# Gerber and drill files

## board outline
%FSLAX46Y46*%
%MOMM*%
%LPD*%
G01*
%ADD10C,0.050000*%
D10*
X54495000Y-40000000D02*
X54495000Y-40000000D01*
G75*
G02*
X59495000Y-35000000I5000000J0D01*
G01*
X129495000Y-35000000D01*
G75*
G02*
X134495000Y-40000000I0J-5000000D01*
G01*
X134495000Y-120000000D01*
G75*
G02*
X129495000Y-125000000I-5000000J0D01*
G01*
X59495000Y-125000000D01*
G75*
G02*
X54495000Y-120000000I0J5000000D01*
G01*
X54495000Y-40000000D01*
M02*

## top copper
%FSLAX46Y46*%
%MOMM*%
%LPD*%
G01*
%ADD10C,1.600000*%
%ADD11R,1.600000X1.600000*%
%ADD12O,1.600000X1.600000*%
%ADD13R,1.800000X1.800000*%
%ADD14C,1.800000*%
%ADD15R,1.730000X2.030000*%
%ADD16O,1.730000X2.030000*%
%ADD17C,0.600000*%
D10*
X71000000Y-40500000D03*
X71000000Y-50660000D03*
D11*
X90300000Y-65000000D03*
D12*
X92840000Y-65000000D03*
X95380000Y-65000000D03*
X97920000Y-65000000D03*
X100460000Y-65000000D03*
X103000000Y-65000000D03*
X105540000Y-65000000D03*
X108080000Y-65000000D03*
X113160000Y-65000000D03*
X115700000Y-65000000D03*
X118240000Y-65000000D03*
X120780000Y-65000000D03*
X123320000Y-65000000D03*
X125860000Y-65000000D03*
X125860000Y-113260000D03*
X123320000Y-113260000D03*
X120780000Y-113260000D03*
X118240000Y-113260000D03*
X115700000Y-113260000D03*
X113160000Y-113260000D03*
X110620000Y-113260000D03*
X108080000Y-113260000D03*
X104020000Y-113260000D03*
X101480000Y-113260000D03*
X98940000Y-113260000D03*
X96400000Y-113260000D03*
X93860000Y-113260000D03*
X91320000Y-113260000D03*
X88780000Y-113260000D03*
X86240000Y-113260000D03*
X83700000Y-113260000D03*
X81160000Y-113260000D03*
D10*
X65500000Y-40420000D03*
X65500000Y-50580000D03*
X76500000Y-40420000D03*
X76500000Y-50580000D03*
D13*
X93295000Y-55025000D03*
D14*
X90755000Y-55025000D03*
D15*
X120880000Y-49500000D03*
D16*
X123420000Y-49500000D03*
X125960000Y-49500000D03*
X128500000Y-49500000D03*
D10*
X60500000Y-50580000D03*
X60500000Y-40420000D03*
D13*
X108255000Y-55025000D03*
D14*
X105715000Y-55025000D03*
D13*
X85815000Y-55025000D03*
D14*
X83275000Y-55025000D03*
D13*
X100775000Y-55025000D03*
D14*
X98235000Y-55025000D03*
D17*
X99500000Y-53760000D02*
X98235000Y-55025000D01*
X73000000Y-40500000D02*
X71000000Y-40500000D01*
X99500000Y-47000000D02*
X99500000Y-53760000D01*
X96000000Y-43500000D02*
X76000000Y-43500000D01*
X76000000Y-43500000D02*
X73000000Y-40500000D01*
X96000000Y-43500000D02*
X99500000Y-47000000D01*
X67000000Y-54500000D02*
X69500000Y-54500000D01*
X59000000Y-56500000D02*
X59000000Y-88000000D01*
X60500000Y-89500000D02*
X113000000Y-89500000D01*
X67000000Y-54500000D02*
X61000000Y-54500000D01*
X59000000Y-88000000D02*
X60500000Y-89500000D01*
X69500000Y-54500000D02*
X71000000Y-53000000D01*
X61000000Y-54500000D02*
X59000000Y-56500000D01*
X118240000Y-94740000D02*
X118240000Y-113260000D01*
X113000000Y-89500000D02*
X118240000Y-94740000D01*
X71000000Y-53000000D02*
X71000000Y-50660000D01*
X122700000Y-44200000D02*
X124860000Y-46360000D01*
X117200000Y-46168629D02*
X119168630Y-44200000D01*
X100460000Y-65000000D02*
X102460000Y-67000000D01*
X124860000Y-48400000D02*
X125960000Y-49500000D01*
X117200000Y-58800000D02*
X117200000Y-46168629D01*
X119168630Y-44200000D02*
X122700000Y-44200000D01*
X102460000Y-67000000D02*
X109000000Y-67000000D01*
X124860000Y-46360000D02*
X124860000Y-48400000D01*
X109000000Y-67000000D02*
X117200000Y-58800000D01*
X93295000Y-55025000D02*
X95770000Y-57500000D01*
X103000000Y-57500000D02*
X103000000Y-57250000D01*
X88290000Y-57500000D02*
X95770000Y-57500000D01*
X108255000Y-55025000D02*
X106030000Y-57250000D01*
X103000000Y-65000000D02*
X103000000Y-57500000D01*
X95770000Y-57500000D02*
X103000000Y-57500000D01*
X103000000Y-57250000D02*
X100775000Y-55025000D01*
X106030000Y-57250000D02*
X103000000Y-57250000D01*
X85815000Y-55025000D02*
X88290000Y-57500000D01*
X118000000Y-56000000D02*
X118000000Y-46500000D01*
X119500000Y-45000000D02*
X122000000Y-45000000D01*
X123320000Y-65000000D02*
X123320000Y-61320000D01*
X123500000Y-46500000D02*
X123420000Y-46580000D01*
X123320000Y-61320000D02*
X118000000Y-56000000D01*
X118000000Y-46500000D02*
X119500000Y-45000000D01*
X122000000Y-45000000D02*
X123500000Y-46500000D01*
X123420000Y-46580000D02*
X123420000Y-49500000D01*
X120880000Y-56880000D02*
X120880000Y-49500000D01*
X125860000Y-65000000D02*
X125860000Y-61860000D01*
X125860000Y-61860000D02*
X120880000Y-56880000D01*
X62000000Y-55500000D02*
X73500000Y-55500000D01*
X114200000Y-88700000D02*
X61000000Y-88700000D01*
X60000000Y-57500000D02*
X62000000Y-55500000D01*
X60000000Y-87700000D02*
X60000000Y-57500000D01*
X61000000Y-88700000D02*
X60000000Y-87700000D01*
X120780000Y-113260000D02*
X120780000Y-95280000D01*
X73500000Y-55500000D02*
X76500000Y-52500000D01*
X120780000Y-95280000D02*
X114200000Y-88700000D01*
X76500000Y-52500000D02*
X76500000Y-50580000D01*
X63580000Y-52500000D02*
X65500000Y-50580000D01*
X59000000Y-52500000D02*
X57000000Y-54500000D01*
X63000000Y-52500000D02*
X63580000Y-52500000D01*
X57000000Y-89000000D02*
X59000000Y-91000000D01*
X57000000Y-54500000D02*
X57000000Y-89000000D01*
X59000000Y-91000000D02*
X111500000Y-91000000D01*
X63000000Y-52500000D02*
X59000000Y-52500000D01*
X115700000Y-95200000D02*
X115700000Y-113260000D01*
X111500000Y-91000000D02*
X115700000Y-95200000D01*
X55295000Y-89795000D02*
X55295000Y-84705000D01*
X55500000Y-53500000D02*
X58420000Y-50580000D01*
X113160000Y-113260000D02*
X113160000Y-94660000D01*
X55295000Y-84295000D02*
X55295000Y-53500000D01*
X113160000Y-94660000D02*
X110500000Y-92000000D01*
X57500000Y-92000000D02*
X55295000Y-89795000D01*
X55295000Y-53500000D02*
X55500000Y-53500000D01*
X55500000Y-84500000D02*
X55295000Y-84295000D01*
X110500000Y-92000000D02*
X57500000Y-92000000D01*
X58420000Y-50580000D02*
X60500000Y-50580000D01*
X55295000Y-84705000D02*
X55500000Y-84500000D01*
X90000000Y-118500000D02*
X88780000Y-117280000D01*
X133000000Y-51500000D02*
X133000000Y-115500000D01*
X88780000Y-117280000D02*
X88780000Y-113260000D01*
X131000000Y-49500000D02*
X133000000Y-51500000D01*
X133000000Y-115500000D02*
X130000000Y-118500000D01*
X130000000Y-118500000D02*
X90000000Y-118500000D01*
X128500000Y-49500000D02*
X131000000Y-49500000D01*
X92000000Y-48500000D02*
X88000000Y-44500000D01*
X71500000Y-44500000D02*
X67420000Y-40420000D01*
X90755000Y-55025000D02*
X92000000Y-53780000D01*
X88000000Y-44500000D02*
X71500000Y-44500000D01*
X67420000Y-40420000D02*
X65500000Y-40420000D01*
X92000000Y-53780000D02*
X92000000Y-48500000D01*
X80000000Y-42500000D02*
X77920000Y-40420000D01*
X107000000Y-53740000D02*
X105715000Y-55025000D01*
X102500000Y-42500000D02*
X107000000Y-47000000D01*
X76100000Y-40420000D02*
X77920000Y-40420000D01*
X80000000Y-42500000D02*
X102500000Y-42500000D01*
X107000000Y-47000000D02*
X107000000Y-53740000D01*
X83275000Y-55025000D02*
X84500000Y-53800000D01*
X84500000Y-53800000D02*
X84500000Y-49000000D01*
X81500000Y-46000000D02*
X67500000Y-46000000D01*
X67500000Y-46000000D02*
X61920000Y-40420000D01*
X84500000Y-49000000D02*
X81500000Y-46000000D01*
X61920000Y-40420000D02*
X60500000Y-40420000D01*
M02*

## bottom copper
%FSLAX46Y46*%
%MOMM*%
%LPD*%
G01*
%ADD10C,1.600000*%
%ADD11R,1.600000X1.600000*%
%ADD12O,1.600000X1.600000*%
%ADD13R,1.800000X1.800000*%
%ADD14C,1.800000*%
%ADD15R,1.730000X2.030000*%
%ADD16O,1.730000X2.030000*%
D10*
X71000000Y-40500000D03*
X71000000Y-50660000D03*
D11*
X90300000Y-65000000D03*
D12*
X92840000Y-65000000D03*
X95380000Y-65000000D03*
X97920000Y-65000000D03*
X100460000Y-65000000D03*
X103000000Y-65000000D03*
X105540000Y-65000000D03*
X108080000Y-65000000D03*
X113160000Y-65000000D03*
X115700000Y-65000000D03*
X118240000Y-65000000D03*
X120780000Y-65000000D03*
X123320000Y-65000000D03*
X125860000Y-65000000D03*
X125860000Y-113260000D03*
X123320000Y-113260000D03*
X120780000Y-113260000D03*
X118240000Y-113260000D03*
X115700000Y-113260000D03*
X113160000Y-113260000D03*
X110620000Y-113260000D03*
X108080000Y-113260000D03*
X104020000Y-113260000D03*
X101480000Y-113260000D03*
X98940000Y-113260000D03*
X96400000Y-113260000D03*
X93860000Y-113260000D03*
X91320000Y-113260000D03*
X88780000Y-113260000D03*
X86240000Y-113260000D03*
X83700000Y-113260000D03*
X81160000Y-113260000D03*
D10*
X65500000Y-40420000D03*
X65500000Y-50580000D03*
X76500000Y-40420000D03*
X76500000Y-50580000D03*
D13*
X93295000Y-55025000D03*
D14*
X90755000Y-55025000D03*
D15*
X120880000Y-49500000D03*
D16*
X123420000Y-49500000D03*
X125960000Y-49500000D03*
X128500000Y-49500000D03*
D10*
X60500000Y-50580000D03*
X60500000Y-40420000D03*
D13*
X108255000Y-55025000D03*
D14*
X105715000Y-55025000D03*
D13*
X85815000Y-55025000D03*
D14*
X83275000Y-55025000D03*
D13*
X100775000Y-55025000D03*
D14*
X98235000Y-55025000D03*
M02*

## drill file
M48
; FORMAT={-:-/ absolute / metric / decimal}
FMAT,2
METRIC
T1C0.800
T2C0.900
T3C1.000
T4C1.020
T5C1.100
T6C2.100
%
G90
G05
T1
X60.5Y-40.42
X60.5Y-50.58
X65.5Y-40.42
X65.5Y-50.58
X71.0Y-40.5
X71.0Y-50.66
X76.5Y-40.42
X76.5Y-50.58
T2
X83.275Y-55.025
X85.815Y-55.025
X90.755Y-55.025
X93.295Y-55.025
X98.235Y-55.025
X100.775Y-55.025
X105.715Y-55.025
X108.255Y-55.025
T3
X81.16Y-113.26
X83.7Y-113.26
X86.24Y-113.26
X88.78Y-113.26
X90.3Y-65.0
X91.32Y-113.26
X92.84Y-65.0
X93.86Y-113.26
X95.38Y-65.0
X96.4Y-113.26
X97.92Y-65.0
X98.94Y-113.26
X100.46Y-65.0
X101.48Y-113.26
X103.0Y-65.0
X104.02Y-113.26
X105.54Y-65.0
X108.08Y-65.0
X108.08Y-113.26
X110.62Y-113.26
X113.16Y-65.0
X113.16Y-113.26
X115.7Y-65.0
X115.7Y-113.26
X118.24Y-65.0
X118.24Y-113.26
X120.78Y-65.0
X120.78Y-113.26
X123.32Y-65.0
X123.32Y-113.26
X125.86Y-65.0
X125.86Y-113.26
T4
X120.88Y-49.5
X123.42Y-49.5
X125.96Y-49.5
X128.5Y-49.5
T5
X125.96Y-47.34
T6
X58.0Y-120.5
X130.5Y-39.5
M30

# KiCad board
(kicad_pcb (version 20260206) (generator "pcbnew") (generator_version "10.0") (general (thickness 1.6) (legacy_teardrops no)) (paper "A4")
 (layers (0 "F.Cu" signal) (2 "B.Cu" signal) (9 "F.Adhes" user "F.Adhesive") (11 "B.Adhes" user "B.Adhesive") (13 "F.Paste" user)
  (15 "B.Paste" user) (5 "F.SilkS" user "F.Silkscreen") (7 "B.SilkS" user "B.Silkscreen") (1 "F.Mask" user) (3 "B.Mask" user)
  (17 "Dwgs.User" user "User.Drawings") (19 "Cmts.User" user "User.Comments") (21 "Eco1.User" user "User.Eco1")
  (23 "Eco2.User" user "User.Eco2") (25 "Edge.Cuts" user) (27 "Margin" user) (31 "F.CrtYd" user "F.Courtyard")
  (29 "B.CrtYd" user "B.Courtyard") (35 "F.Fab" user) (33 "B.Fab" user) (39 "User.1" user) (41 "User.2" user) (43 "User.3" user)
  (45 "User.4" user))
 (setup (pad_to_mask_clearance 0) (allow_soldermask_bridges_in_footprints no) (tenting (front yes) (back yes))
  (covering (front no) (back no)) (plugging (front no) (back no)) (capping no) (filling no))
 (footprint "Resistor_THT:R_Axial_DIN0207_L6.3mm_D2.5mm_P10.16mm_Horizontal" (layer "F.Cu") (at 71 40.5 -90)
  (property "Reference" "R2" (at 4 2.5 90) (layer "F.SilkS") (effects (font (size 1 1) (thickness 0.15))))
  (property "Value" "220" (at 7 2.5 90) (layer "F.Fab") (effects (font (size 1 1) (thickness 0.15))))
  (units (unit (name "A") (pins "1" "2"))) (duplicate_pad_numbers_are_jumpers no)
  (pad "1" thru_hole circle (at 0 0 270) (size 1.6 1.6) (drill 0.8) (layers "*.Cu" "*.Mask") (remove_unused_layers no) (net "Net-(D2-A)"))
  (pad "2" thru_hole circle (at 10.16 0 270) (size 1.6 1.6) (drill 0.8) (layers "*.Cu" "*.Mask") (remove_unused_layers no)
   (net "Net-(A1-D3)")))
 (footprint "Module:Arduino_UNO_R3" (layer "F.Cu") (at 90.3 65)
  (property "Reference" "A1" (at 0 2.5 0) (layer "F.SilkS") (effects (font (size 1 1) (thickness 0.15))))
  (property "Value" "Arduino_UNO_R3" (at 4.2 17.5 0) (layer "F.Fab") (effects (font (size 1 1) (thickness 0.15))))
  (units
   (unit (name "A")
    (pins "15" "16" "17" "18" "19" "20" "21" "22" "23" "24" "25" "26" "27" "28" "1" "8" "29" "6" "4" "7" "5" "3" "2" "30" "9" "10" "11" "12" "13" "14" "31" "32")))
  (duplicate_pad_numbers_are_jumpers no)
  (pad "1" thru_hole rect (at 0 0 90) (size 1.6 1.6) (drill 1) (layers "*.Cu" "*.Mask") (remove_unused_layers no)
   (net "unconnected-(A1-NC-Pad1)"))
  (pad "2" thru_hole oval (at 2.54 0 90) (size 1.6 1.6) (drill 1) (layers "*.Cu" "*.Mask") (remove_unused_layers no)
   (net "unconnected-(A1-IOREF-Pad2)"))
  (pad "3" thru_hole oval (at 5.08 0 90) (size 1.6 1.6) (drill 1) (layers "*.Cu" "*.Mask") (remove_unused_layers no)
   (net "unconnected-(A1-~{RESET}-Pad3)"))
  (pad "4" thru_hole oval (at 7.62 0 90) (size 1.6 1.6) (drill 1) (layers "*.Cu" "*.Mask") (remove_unused_layers no)
   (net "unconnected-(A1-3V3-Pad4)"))
  (pad "5" thru_hole oval (at 10.16 0 90) (size 1.6 1.6) (drill 1) (layers "*.Cu" "*.Mask") (remove_unused_layers no) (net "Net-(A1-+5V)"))
  (pad "6" thru_hole oval (at 12.7 0 90) (size 1.6 1.6) (drill 1) (layers "*.Cu" "*.Mask") (remove_unused_layers no) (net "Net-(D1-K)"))
  (pad "7" thru_hole oval (at 15.24 0 90) (size 1.6 1.6) (drill 1) (layers "*.Cu" "*.Mask") (remove_unused_layers no)
   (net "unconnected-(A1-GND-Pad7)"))
  (pad "8" thru_hole oval (at 17.78 0 90) (size 1.6 1.6) (drill 1) (layers "*.Cu" "*.Mask") (remove_unused_layers no)
   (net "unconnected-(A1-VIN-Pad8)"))
  (pad "9" thru_hole oval (at 22.86 0 90) (size 1.6 1.6) (drill 1) (layers "*.Cu" "*.Mask") (remove_unused_layers no)
   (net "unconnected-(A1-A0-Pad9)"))
  (pad "10" thru_hole oval (at 25.4 0 90) (size 1.6 1.6) (drill 1) (layers "*.Cu" "*.Mask") (remove_unused_layers no)
   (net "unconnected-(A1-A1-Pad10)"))
  (pad "11" thru_hole oval (at 27.94 0 90) (size 1.6 1.6) (drill 1) (layers "*.Cu" "*.Mask") (remove_unused_layers no)
   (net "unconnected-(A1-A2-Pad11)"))
  (pad "12" thru_hole oval (at 30.48 0 90) (size 1.6 1.6) (drill 1) (layers "*.Cu" "*.Mask") (remove_unused_layers no)
   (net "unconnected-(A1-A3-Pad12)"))
  (pad "13" thru_hole oval (at 33.02 0 90) (size 1.6 1.6) (drill 1) (layers "*.Cu" "*.Mask") (remove_unused_layers no)
   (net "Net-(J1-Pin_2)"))
  (pad "14" thru_hole oval (at 35.56 0 90) (size 1.6 1.6) (drill 1) (layers "*.Cu" "*.Mask") (remove_unused_layers no)
   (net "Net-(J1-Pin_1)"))
  (pad "15" thru_hole oval (at 35.56 48.26 90) (size 1.6 1.6) (drill 1) (layers "*.Cu" "*.Mask") (remove_unused_layers no)
   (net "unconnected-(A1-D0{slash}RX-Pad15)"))
  (pad "16" thru_hole oval (at 33.02 48.26 90) (size 1.6 1.6) (drill 1) (layers "*.Cu" "*.Mask") (remove_unused_layers no)
   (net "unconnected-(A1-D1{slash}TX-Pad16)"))
  (pad "17" thru_hole oval (at 30.48 48.26 90) (size 1.6 1.6) (drill 1) (layers "*.Cu" "*.Mask") (remove_unused_layers no)
   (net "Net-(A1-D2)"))
  (pad "18" thru_hole oval (at 27.94 48.26 90) (size 1.6 1.6) (drill 1) (layers "*.Cu" "*.Mask") (remove_unused_layers no)
   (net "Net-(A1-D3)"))
  (pad "19" thru_hole oval (at 25.4 48.26 90) (size 1.6 1.6) (drill 1) (layers "*.Cu" "*.Mask") (remove_unused_layers no)
   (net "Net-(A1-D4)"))
  (pad "20" thru_hole oval (at 22.86 48.26 90) (size 1.6 1.6) (drill 1) (layers "*.Cu" "*.Mask") (remove_unused_layers no)
   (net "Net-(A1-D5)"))
  (pad "21" thru_hole oval (at 20.32 48.26 90) (size 1.6 1.6) (drill 1) (layers "*.Cu" "*.Mask") (remove_unused_layers no)
   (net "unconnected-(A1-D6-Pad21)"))
  (pad "22" thru_hole oval (at 17.78 48.26 90) (size 1.6 1.6) (drill 1) (layers "*.Cu" "*.Mask") (remove_unused_layers no)
   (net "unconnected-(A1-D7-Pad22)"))
  (pad "23" thru_hole oval (at 13.72 48.26 90) (size 1.6 1.6) (drill 1) (layers "*.Cu" "*.Mask") (remove_unused_layers no)
   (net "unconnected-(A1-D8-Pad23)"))
  (pad "24" thru_hole oval (at 11.18 48.26 90) (size 1.6 1.6) (drill 1) (layers "*.Cu" "*.Mask") (remove_unused_layers no)
   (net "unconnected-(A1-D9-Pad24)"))
  (pad "25" thru_hole oval (at 8.64 48.26 90) (size 1.6 1.6) (drill 1) (layers "*.Cu" "*.Mask") (remove_unused_layers no)
   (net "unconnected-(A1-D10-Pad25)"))
  (pad "26" thru_hole oval (at 6.1 48.26 90) (size 1.6 1.6) (drill 1) (layers "*.Cu" "*.Mask") (remove_unused_layers no)
   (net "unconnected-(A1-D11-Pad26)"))
  (pad "27" thru_hole oval (at 3.56 48.26 90) (size 1.6 1.6) (drill 1) (layers "*.Cu" "*.Mask") (remove_unused_layers no)
   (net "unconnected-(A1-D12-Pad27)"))
  (pad "28" thru_hole oval (at 1.02 48.26 90) (size 1.6 1.6) (drill 1) (layers "*.Cu" "*.Mask") (remove_unused_layers no)
   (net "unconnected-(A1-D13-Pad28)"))
  (pad "29" thru_hole oval (at -1.52 48.26 90) (size 1.6 1.6) (drill 1) (layers "*.Cu" "*.Mask") (remove_unused_layers no)
   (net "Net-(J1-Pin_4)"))
  (pad "30" thru_hole oval (at -4.06 48.26 90) (size 1.6 1.6) (drill 1) (layers "*.Cu" "*.Mask") (remove_unused_layers no)
   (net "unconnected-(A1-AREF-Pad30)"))
  (pad "31" thru_hole oval (at -6.6 48.26 90) (size 1.6 1.6) (drill 1) (layers "*.Cu" "*.Mask") (remove_unused_layers no)
   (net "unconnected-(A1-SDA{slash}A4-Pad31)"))
  (pad "32" thru_hole oval (at -9.14 48.26 90) (size 1.6 1.6) (drill 1) (layers "*.Cu" "*.Mask") (remove_unused_layers no)
   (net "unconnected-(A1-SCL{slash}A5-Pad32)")))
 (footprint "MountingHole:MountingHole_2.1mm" (layer "F.Cu") (at 58 120.5)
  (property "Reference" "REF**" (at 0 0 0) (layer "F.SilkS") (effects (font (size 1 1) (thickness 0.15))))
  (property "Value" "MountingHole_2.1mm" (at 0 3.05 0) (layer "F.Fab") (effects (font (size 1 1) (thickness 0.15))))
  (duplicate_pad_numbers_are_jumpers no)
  (pad "" np_thru_hole circle (at 0 0) (size 2.1 2.1) (drill 2.1) (layers "*.Cu" "*.Mask")))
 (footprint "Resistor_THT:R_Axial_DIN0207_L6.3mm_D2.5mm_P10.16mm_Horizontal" (layer "F.Cu") (at 65.5 40.42 -90)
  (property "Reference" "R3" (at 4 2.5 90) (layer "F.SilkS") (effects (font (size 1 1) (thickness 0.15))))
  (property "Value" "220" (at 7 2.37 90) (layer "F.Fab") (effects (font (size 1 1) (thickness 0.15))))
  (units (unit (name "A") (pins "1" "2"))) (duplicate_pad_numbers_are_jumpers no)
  (pad "1" thru_hole circle (at 0 0 270) (size 1.6 1.6) (drill 0.8) (layers "*.Cu" "*.Mask") (remove_unused_layers no) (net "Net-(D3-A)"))
  (pad "2" thru_hole circle (at 10.16 0 270) (size 1.6 1.6) (drill 0.8) (layers "*.Cu" "*.Mask") (remove_unused_layers no)
   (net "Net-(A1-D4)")))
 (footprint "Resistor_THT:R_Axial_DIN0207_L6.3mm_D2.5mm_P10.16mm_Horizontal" (layer "F.Cu") (at 76.5 40.42 -90)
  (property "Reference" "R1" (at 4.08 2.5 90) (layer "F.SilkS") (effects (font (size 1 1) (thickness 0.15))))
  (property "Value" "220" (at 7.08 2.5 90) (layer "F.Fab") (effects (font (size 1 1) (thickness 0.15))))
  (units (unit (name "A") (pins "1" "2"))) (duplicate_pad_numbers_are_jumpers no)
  (pad "1" thru_hole circle (at 0 0 270) (size 1.6 1.6) (drill 0.8) (layers "*.Cu" "*.Mask") (remove_unused_layers no) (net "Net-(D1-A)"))
  (pad "2" thru_hole circle (at 10.16 0 270) (size 1.6 1.6) (drill 0.8) (layers "*.Cu" "*.Mask") (remove_unused_layers no)
   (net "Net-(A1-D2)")))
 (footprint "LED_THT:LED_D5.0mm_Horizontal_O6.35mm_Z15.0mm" (layer "F.Cu") (at 93.295 55.025 180)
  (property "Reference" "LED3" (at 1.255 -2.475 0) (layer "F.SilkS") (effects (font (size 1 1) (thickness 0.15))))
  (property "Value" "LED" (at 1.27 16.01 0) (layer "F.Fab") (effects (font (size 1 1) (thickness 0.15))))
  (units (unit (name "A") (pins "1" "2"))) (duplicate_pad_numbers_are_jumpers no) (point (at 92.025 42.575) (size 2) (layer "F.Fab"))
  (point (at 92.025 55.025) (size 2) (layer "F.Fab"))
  (pad "1" thru_hole rect (at 0 0 180) (size 1.8 1.8) (drill 0.9) (layers "*.Cu" "*.Mask") (remove_unused_layers no) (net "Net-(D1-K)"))
  (pad "2" thru_hole circle (at 2.54 0 180) (size 1.8 1.8) (drill 0.9) (layers "*.Cu" "*.Mask") (remove_unused_layers no) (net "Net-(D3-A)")))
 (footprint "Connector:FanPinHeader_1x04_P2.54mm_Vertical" (layer "F.Cu") (at 120.88 49.5)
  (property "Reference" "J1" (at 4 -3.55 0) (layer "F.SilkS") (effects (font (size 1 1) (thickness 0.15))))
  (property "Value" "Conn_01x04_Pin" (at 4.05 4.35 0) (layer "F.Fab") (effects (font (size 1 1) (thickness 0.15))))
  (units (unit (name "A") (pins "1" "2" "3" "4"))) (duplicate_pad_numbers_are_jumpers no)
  (pad "" np_thru_hole circle (at 5.08 -2.16 90) (size 1.1 1.1) (drill 1.1) (layers "*.Cu" "*.Mask"))
  (pad "1" thru_hole rect (at 0 0 90) (size 2.03 1.73) (drill 1.02) (layers "*.Cu" "*.Mask") (remove_unused_layers no)
   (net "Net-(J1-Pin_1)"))
  (pad "2" thru_hole oval (at 2.54 0 90) (size 2.03 1.73) (drill 1.02) (layers "*.Cu" "*.Mask") (remove_unused_layers no)
   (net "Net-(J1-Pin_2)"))
  (pad "3" thru_hole oval (at 5.08 0 90) (size 2.03 1.73) (drill 1.02) (layers "*.Cu" "*.Mask") (remove_unused_layers no)
   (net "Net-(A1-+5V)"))
  (pad "4" thru_hole oval (at 7.62 0 90) (size 2.03 1.73) (drill 1.02) (layers "*.Cu" "*.Mask") (remove_unused_layers no)
   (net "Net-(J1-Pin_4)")))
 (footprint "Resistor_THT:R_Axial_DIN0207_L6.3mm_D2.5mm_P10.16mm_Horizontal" (layer "F.Cu") (at 60.5 50.58 90)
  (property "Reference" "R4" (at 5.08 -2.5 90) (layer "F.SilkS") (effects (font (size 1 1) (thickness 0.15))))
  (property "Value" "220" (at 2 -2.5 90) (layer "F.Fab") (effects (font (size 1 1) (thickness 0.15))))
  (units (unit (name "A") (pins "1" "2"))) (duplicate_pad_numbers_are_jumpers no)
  (pad "1" thru_hole circle (at 0 0 90) (size 1.6 1.6) (drill 0.8) (layers "*.Cu" "*.Mask") (remove_unused_layers no) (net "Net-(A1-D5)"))
  (pad "2" thru_hole circle (at 10.16 0 90) (size 1.6 1.6) (drill 0.8) (layers "*.Cu" "*.Mask") (remove_unused_layers no) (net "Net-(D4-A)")))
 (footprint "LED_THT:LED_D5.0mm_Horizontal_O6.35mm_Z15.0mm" (layer "F.Cu") (at 108.255 55.025 180)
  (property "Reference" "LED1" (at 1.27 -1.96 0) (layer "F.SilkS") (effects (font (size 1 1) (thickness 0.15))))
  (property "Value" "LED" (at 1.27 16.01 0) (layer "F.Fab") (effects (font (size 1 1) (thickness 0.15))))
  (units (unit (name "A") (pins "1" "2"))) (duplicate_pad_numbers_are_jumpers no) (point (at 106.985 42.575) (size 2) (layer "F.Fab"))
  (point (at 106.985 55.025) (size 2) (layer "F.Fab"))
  (pad "1" thru_hole rect (at 0 0 180) (size 1.8 1.8) (drill 0.9) (layers "*.Cu" "*.Mask") (remove_unused_layers no) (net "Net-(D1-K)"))
  (pad "2" thru_hole circle (at 2.54 0 180) (size 1.8 1.8) (drill 0.9) (layers "*.Cu" "*.Mask") (remove_unused_layers no) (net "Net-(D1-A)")))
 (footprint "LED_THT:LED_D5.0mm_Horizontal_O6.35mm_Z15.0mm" (layer "F.Cu") (at 85.815 55.025 180)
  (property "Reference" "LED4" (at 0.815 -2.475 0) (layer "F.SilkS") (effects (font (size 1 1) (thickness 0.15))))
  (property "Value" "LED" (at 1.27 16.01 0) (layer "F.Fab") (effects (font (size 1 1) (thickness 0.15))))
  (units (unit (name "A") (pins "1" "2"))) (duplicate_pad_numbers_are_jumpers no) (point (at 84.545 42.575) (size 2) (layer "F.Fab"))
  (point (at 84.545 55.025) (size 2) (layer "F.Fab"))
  (pad "1" thru_hole rect (at 0 0 180) (size 1.8 1.8) (drill 0.9) (layers "*.Cu" "*.Mask") (remove_unused_layers no) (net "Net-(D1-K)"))
  (pad "2" thru_hole circle (at 2.54 0 180) (size 1.8 1.8) (drill 0.9) (layers "*.Cu" "*.Mask") (remove_unused_layers no) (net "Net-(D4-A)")))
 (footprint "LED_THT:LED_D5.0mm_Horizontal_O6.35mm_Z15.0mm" (layer "F.Cu") (at 100.775 55.025 180)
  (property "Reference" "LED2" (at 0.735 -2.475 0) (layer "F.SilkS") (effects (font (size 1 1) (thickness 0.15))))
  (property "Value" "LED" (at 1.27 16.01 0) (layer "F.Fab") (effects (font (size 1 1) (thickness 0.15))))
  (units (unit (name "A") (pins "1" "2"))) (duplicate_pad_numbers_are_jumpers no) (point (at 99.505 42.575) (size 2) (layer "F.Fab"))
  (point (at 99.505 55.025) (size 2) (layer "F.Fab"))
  (pad "1" thru_hole rect (at 0 0 180) (size 1.8 1.8) (drill 0.9) (layers "*.Cu" "*.Mask") (remove_unused_layers no) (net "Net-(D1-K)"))
  (pad "2" thru_hole circle (at 2.54 0 180) (size 1.8 1.8) (drill 0.9) (layers "*.Cu" "*.Mask") (remove_unused_layers no) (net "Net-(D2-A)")))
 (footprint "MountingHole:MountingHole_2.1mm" (layer "F.Cu") (at 130.5 39.5)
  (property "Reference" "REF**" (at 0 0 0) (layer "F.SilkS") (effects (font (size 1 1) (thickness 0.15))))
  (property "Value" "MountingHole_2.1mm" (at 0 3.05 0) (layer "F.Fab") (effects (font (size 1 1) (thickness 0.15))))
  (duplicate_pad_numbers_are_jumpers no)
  (pad "" np_thru_hole circle (at 0 0) (size 2.1 2.1) (drill 2.1) (layers "*.Cu" "*.Mask")))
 (gr_rect (start 54.495 35) (end 134.495 125) (radius 5) (stroke (width 0.05) (type solid)) (fill no) (layer "Edge.Cuts"))
 (segment (start 99.5 53.76) (end 98.235 55.025) (width 0.6) (layer "F.Cu") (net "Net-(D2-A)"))
 (segment (start 73 40.5) (end 71 40.5) (width 0.6) (layer "F.Cu") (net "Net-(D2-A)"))
 (segment (start 99.5 47) (end 99.5 53.76) (width 0.6) (layer "F.Cu") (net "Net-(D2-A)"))
 (segment (start 96 43.5) (end 76 43.5) (width 0.6) (layer "F.Cu") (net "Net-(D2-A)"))
 (segment (start 76 43.5) (end 73 40.5) (width 0.6) (layer "F.Cu") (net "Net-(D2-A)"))
 (segment (start 96 43.5) (end 99.5 47) (width 0.6) (layer "F.Cu") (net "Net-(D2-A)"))
 (segment (start 67 54.5) (end 69.5 54.5) (width 0.6) (layer "F.Cu") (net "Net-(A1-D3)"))
 (segment (start 59 56.5) (end 59 88) (width 0.6) (layer "F.Cu") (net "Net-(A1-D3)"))
 (segment (start 60.5 89.5) (end 113 89.5) (width 0.6) (layer "F.Cu") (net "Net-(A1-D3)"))
 (segment (start 67 54.5) (end 61 54.5) (width 0.6) (layer "F.Cu") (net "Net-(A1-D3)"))
 (segment (start 59 88) (end 60.5 89.5) (width 0.6) (layer "F.Cu") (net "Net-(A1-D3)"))
 (segment (start 69.5 54.5) (end 71 53) (width 0.6) (layer "F.Cu") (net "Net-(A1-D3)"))
 (segment (start 61 54.5) (end 59 56.5) (width 0.6) (layer "F.Cu") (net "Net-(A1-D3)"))
 (segment (start 118.24 94.74) (end 118.24 113.26) (width 0.6) (layer "F.Cu") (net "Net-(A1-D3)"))
 (segment (start 113 89.5) (end 118.24 94.74) (width 0.6) (layer "F.Cu") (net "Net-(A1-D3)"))
 (segment (start 71 53) (end 71 50.66) (width 0.6) (layer "F.Cu") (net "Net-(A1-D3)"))
 (segment (start 122.7 44.2) (end 124.86 46.36) (width 0.6) (layer "F.Cu") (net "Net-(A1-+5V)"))
 (segment (start 117.2 46.168629) (end 119.16863 44.2) (width 0.6) (layer "F.Cu") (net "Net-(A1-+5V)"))
 (segment (start 100.46 65) (end 102.46 67) (width 0.6) (layer "F.Cu") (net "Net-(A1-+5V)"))
 (segment (start 124.86 48.4) (end 125.96 49.5) (width 0.6) (layer "F.Cu") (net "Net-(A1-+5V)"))
 (segment (start 117.2 58.8) (end 117.2 46.168629) (width 0.6) (layer "F.Cu") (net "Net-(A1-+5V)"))
 (segment (start 119.16863 44.2) (end 122.7 44.2) (width 0.6) (layer "F.Cu") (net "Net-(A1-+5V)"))
 (segment (start 102.46 67) (end 109 67) (width 0.6) (layer "F.Cu") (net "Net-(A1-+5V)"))
 (segment (start 124.86 46.36) (end 124.86 48.4) (width 0.6) (layer "F.Cu") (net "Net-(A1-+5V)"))
 (segment (start 109 67) (end 117.2 58.8) (width 0.6) (layer "F.Cu") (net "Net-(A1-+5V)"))
 (segment (start 93.295 55.025) (end 95.77 57.5) (width 0.6) (layer "F.Cu") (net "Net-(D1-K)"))
 (segment (start 103 57.5) (end 103 57.25) (width 0.6) (layer "F.Cu") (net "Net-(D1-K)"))
 (segment (start 88.29 57.5) (end 95.77 57.5) (width 0.6) (layer "F.Cu") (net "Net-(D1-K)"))
 (segment (start 108.255 55.025) (end 106.03 57.25) (width 0.6) (layer "F.Cu") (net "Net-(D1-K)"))
 (segment (start 103 65) (end 103 57.5) (width 0.6) (layer "F.Cu") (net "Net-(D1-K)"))
 (segment (start 95.77 57.5) (end 103 57.5) (width 0.6) (layer "F.Cu") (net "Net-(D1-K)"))
 (segment (start 103 57.25) (end 100.775 55.025) (width 0.6) (layer "F.Cu") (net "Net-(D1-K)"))
 (segment (start 106.03 57.25) (end 103 57.25) (width 0.6) (layer "F.Cu") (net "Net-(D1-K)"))
 (segment (start 85.815 55.025) (end 88.29 57.5) (width 0.6) (layer "F.Cu") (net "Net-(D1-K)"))
 (segment (start 118 56) (end 118 46.5) (width 0.6) (layer "F.Cu") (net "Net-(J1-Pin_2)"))
 (segment (start 119.5 45) (end 122 45) (width 0.6) (layer "F.Cu") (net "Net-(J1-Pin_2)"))
 (segment (start 123.32 65) (end 123.32 61.32) (width 0.6) (layer "F.Cu") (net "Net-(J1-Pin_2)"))
 (segment (start 123.5 46.5) (end 123.42 46.58) (width 0.6) (layer "F.Cu") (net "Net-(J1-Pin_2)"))
 (segment (start 123.32 61.32) (end 118 56) (width 0.6) (layer "F.Cu") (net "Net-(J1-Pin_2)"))
 (segment (start 118 46.5) (end 119.5 45) (width 0.6) (layer "F.Cu") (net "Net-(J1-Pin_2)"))
 (segment (start 122 45) (end 123.5 46.5) (width 0.6) (layer "F.Cu") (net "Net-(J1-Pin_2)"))
 (segment (start 123.42 46.58) (end 123.42 49.5) (width 0.6) (layer "F.Cu") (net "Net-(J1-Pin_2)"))
 (segment (start 120.88 56.88) (end 120.88 49.5) (width 0.6) (layer "F.Cu") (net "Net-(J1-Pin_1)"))
 (segment (start 125.86 65) (end 125.86 61.86) (width 0.6) (layer "F.Cu") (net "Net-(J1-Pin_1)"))
 (segment (start 125.86 61.86) (end 120.88 56.88) (width 0.6) (layer "F.Cu") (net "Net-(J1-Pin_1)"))
 (segment (start 62 55.5) (end 73.5 55.5) (width 0.6) (layer "F.Cu") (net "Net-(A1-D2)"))
 (segment (start 114.2 88.7) (end 61 88.7) (width 0.6) (layer "F.Cu") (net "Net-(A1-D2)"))
 (segment (start 60 57.5) (end 62 55.5) (width 0.6) (layer "F.Cu") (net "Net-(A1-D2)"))
 (segment (start 60 87.7) (end 60 57.5) (width 0.6) (layer "F.Cu") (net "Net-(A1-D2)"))
 (segment (start 61 88.7) (end 60 87.7) (width 0.6) (layer "F.Cu") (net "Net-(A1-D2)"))
 (segment (start 120.78 113.26) (end 120.78 95.28) (width 0.6) (layer "F.Cu") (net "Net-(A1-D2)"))
 (segment (start 73.5 55.5) (end 76.5 52.5) (width 0.6) (layer "F.Cu") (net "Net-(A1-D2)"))
 (segment (start 120.78 95.28) (end 114.2 88.7) (width 0.6) (layer "F.Cu") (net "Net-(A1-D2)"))
 (segment (start 76.5 52.5) (end 76.5 50.58) (width 0.6) (layer "F.Cu") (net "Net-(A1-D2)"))
 (segment (start 63.58 52.5) (end 65.5 50.58) (width 0.6) (layer "F.Cu") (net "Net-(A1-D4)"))
 (segment (start 59 52.5) (end 57 54.5) (width 0.6) (layer "F.Cu") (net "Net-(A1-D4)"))
 (segment (start 63 52.5) (end 63.58 52.5) (width 0.6) (layer "F.Cu") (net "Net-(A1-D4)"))
 (segment (start 57 89) (end 59 91) (width 0.6) (layer "F.Cu") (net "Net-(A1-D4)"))
 (segment (start 57 54.5) (end 57 89) (width 0.6) (layer "F.Cu") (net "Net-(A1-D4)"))
 (segment (start 59 91) (end 111.5 91) (width 0.6) (layer "F.Cu") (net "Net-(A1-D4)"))
 (segment (start 63 52.5) (end 59 52.5) (width 0.6) (layer "F.Cu") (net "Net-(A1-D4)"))
 (segment (start 115.7 95.2) (end 115.7 113.26) (width 0.6) (layer "F.Cu") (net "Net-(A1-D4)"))
 (segment (start 111.5 91) (end 115.7 95.2) (width 0.6) (layer "F.Cu") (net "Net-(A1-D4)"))
 (segment (start 55.295 89.795) (end 55.295 84.705) (width 0.6) (layer "F.Cu") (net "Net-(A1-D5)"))
 (segment (start 55.5 53.5) (end 58.42 50.58) (width 0.6) (layer "F.Cu") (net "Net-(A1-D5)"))
 (segment (start 113.16 113.26) (end 113.16 94.66) (width 0.6) (layer "F.Cu") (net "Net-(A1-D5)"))
 (segment (start 55.295 84.295) (end 55.295 53.5) (width 0.6) (layer "F.Cu") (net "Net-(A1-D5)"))
 (segment (start 113.16 94.66) (end 110.5 92) (width 0.6) (layer "F.Cu") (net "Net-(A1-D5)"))
 (segment (start 57.5 92) (end 55.295 89.795) (width 0.6) (layer "F.Cu") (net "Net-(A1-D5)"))
 (segment (start 55.295 53.5) (end 55.5 53.5) (width 0.6) (layer "F.Cu") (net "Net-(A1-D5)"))
 (segment (start 55.5 84.5) (end 55.295 84.295) (width 0.6) (layer "F.Cu") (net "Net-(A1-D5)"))
 (segment (start 110.5 92) (end 57.5 92) (width 0.6) (layer "F.Cu") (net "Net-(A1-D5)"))
 (segment (start 58.42 50.58) (end 60.5 50.58) (width 0.6) (layer "F.Cu") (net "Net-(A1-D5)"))
 (segment (start 55.295 84.705) (end 55.5 84.5) (width 0.6) (layer "F.Cu") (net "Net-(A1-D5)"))
 (segment (start 90 118.5) (end 88.78 117.28) (width 0.6) (layer "F.Cu") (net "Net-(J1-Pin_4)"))
 (segment (start 133 51.5) (end 133 115.5) (width 0.6) (layer "F.Cu") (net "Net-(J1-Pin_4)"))
 (segment (start 88.78 117.28) (end 88.78 113.26) (width 0.6) (layer "F.Cu") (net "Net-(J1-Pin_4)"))
 (segment (start 131 49.5) (end 133 51.5) (width 0.6) (layer "F.Cu") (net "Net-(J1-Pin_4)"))
 (segment (start 133 115.5) (end 130 118.5) (width 0.6) (layer "F.Cu") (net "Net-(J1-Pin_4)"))
 (segment (start 130 118.5) (end 90 118.5) (width 0.6) (layer "F.Cu") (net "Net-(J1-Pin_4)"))
 (segment (start 128.5 49.5) (end 131 49.5) (width 0.6) (layer "F.Cu") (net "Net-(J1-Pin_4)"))
 (segment (start 92 48.5) (end 88 44.5) (width 0.6) (layer "F.Cu") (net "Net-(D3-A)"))
 (segment (start 71.5 44.5) (end 67.42 40.42) (width 0.6) (layer "F.Cu") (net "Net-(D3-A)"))
 (segment (start 90.755 55.025) (end 92 53.78) (width 0.6) (layer "F.Cu") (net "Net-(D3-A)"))
 (segment (start 88 44.5) (end 71.5 44.5) (width 0.6) (layer "F.Cu") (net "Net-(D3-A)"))
 (segment (start 67.42 40.42) (end 65.5 40.42) (width 0.6) (layer "F.Cu") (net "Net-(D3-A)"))
 (segment (start 92 53.78) (end 92 48.5) (width 0.6) (layer "F.Cu") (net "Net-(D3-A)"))
 (segment (start 80 42.5) (end 77.92 40.42) (width 0.6) (layer "F.Cu") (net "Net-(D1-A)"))
 (segment (start 107 53.74) (end 105.715 55.025) (width 0.6) (layer "F.Cu") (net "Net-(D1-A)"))
 (segment (start 102.5 42.5) (end 107 47) (width 0.6) (layer "F.Cu") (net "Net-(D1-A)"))
 (segment (start 76.1 40.42) (end 77.92 40.42) (width 0.6) (layer "F.Cu") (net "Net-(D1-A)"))
 (segment (start 80 42.5) (end 102.5 42.5) (width 0.6) (layer "F.Cu") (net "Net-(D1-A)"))
 (segment (start 107 47) (end 107 53.74) (width 0.6) (layer "F.Cu") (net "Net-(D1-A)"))
 (segment (start 83.275 55.025) (end 84.5 53.8) (width 0.6) (layer "F.Cu") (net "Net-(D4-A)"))
 (segment (start 84.5 53.8) (end 84.5 49) (width 0.6) (layer "F.Cu") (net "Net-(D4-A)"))
 (segment (start 81.5 46) (end 67.5 46) (width 0.6) (layer "F.Cu") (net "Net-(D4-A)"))
 (segment (start 67.5 46) (end 61.92 40.42) (width 0.6) (layer "F.Cu") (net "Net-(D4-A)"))
 (segment (start 84.5 49) (end 81.5 46) (width 0.6) (layer "F.Cu") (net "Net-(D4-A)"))
 (segment (start 61.92 40.42) (end 60.5 40.42) (width 0.6) (layer "F.Cu") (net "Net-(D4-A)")))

